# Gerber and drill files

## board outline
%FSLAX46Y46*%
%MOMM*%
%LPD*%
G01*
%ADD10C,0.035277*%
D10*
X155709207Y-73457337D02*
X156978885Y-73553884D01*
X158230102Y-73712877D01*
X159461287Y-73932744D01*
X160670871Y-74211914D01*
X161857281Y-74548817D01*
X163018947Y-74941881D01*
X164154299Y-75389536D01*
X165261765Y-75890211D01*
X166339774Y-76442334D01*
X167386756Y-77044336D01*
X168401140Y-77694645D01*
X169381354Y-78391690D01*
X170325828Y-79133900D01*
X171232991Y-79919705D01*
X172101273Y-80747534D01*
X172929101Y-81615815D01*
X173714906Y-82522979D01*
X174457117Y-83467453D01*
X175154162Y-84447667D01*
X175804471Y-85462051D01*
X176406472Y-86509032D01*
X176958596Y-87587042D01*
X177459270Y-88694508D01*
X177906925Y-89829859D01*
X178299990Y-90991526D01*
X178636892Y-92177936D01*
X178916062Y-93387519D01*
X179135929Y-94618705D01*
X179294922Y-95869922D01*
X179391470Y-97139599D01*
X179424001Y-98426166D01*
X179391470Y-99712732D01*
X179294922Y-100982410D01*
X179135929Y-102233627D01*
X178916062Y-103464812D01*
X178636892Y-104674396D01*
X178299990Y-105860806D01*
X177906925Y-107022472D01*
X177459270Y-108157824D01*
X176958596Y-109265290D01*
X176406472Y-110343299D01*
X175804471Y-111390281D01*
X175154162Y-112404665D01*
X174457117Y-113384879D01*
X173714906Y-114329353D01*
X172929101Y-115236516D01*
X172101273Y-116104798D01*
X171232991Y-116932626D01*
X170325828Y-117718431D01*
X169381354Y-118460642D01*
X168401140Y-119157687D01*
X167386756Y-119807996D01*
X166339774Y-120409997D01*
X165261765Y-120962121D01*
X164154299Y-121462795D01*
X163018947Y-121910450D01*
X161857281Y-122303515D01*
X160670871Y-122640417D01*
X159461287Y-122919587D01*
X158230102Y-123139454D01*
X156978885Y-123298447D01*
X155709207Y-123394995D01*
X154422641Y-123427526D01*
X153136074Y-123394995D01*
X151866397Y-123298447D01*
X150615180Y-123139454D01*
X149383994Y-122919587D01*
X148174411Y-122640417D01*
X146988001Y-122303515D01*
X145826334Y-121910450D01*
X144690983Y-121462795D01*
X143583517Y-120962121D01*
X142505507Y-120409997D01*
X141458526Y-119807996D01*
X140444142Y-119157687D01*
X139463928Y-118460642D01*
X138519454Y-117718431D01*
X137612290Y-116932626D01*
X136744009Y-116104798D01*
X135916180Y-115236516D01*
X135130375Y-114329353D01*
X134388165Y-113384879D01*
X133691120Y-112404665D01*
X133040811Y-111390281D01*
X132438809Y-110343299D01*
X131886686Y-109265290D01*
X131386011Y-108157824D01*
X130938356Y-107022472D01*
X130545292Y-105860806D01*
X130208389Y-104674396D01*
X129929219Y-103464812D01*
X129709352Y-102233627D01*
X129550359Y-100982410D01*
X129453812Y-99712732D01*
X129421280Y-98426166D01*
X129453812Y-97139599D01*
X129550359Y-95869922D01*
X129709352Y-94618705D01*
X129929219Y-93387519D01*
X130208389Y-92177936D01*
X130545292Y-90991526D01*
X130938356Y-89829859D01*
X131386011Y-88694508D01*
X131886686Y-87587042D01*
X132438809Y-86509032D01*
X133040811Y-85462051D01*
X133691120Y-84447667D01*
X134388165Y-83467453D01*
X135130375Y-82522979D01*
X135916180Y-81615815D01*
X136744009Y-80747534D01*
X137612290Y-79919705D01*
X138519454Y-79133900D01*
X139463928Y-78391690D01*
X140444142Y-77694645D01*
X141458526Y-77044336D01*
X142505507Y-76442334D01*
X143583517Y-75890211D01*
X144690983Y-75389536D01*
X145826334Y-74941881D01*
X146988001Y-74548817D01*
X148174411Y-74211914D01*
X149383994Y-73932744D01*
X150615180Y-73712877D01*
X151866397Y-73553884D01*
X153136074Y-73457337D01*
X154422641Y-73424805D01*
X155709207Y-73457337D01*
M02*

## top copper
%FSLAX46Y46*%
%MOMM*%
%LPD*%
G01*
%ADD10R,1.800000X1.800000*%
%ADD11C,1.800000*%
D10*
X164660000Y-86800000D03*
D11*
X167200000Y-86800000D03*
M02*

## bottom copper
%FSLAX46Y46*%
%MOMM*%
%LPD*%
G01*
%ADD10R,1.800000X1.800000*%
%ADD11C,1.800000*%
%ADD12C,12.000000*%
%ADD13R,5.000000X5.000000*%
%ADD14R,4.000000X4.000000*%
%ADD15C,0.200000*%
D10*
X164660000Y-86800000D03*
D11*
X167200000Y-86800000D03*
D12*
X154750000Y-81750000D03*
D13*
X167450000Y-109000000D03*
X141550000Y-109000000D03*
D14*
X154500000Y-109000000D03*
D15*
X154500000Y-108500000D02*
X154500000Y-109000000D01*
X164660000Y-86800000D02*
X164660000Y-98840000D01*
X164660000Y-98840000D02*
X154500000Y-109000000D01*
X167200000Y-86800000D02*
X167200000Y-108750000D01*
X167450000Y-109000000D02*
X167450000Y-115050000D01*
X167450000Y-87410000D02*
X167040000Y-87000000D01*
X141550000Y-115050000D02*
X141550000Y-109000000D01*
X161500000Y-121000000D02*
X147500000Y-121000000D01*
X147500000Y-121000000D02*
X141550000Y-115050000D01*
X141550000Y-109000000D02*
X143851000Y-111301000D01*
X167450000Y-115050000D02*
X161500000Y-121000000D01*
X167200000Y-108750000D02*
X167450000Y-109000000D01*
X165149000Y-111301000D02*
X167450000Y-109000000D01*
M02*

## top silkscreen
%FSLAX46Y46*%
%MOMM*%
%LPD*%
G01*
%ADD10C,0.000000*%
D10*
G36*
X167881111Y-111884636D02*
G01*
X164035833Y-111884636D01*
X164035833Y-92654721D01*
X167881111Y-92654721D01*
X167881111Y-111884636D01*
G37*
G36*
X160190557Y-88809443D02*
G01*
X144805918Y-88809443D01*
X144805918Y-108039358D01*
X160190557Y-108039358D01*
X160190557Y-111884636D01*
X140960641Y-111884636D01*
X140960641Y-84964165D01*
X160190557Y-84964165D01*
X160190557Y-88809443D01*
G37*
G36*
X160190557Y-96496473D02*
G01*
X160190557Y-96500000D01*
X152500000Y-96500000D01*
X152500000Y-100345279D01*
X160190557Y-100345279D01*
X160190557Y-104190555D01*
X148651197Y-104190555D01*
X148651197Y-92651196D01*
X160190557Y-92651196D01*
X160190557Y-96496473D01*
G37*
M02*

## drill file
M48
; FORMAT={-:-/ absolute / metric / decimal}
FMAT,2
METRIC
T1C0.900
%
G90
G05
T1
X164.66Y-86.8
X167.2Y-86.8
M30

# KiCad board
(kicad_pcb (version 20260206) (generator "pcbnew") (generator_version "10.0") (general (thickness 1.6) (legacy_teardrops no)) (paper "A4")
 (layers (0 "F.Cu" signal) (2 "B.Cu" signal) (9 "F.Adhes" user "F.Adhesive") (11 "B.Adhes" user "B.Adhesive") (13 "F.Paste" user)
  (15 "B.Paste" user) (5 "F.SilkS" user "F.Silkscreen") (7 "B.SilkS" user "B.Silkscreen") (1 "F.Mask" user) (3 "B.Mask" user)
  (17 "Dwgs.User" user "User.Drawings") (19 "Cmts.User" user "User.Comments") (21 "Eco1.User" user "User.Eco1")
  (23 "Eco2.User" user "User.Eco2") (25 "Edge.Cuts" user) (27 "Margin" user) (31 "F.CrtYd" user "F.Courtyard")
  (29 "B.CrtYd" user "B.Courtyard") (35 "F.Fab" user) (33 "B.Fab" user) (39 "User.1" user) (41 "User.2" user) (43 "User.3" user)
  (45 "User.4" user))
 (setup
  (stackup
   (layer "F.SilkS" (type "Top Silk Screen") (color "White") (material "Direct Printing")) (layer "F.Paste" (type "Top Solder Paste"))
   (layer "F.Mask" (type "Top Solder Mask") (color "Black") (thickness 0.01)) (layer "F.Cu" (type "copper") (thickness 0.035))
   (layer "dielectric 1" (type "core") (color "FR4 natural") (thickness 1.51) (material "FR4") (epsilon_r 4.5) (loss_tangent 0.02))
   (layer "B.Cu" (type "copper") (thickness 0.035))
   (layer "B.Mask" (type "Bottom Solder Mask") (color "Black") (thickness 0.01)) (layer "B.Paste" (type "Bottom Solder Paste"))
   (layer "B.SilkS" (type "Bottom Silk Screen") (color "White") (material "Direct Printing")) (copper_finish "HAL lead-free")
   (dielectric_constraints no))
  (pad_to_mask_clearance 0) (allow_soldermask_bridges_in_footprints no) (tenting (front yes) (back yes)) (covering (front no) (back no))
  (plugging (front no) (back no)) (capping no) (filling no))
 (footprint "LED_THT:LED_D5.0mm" (layer "F.Cu") (at 164.66 86.8)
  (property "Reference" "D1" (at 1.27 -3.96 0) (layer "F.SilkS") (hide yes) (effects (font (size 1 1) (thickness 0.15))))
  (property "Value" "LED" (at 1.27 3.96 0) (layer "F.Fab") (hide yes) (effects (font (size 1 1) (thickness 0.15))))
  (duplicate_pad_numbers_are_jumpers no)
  (pad "1" thru_hole rect (at 0 0) (size 1.8 1.8) (drill 0.9) (layers "*.Cu" "*.Mask") (remove_unused_layers no) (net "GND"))
  (pad "2" thru_hole circle (at 2.54 0) (size 1.8 1.8) (drill 0.9) (layers "*.Cu" "*.Mask") (remove_unused_layers no) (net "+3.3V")))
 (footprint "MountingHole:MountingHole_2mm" (layer "B.Cu") (at 154.75 81.75 180)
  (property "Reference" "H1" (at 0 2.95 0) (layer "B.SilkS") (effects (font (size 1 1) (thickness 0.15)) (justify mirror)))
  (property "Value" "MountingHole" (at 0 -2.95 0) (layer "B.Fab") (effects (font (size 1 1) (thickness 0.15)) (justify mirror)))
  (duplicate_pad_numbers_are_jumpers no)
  (pad "" smd circle (at 0 0 180) (size 12 12) (layers "B.Cu" "B.Mask" "B.Paste") (thermal_bridge_angle 90)))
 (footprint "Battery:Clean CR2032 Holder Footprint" (layer "B.Cu") (at 154.5 109 180)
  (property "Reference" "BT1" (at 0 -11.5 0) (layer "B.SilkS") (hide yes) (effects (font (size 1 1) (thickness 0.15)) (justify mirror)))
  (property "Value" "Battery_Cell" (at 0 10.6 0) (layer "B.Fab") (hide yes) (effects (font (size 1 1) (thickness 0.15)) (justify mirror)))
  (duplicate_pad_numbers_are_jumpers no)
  (pad "1" smd rect (at -12.95 0 180) (size 5 5) (layers "B.Cu" "B.Mask" "B.Paste") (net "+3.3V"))
  (pad "1" smd rect (at 12.95 0 180) (size 5 5) (layers "B.Cu" "B.Mask" "B.Paste") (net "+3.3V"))
  (pad "2" smd rect (at 0 0 180) (size 4 4) (layers "B.Cu" "B.Mask" "B.Paste") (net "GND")))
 (gr_poly
  (pts (xy 167.881111 111.884636) (xy 164.035833 111.884636) (xy 164.035833 92.654721) (xy 167.881111 92.654721))
  (stroke (width 0) (type solid)) (fill yes) (layer "F.SilkS"))
 (gr_poly
  (pts (xy 160.190557 88.809443) (xy 144.805918 88.809443) (xy 144.805918 108.039358) (xy 160.190557 108.039358) (xy 160.190557 111.884636)
   (xy 140.960641 111.884636) (xy 140.960641 84.964165) (xy 160.190557 84.964165))
  (stroke (width 0) (type solid)) (fill yes) (layer "F.SilkS"))
 (gr_poly
  (pts (xy 160.190557 96.496473) (xy 160.190557 96.5) (xy 152.5 96.5) (xy 152.5 100.345279) (xy 160.190557 100.345279)
   (xy 160.190557 104.190555) (xy 148.651197 104.190555) (xy 148.651197 92.651196) (xy 160.190557 92.651196))
  (stroke (width 0) (type solid)) (fill yes) (layer "F.SilkS"))
 (gr_poly
  (pts (xy 155.709207 73.457337) (xy 156.978885 73.553884) (xy 158.230102 73.712877) (xy 159.461287 73.932744) (xy 160.670871 74.211914)
   (xy 161.857281 74.548817) (xy 163.018947 74.941881) (xy 164.154299 75.389536) (xy 165.261765 75.890211) (xy 166.339774 76.442334)
   (xy 167.386756 77.044336) (xy 168.40114 77.694645) (xy 169.381354 78.39169) (xy 170.325828 79.1339) (xy 171.232991 79.919705)
   (xy 172.101273 80.747534) (xy 172.929101 81.615815) (xy 173.714906 82.522979) (xy 174.457117 83.467453) (xy 175.154162 84.447667)
   (xy 175.804471 85.462051) (xy 176.406472 86.509032) (xy 176.958596 87.587042) (xy 177.45927 88.694508) (xy 177.906925 89.829859)
   (xy 178.29999 90.991526) (xy 178.636892 92.177936) (xy 178.916062 93.387519) (xy 179.135929 94.618705) (xy 179.294922 95.869922)
   (xy 179.39147 97.139599) (xy 179.424001 98.426166) (xy 179.39147 99.712732) (xy 179.294922 100.98241) (xy 179.135929 102.233627)
   (xy 178.916062 103.464812) (xy 178.636892 104.674396) (xy 178.29999 105.860806) (xy 177.906925 107.022472) (xy 177.45927 108.157824)
   (xy 176.958596 109.26529) (xy 176.406472 110.343299) (xy 175.804471 111.390281) (xy 175.154162 112.404665) (xy 174.457117 113.384879)
   (xy 173.714906 114.329353) (xy 172.929101 115.236516) (xy 172.101273 116.104798) (xy 171.232991 116.932626) (xy 170.325828 117.718431)
   (xy 169.381354 118.460642) (xy 168.40114 119.157687) (xy 167.386756 119.807996) (xy 166.339774 120.409997) (xy 165.261765 120.962121)
   (xy 164.154299 121.462795) (xy 163.018947 121.91045) (xy 161.857281 122.303515) (xy 160.670871 122.640417) (xy 159.461287 122.919587)
   (xy 158.230102 123.139454) (xy 156.978885 123.298447) (xy 155.709207 123.394995) (xy 154.422641 123.427526) (xy 153.136074 123.394995)
   (xy 151.866397 123.298447) (xy 150.61518 123.139454) (xy 149.383994 122.919587) (xy 148.174411 122.640417) (xy 146.988001 122.303515)
   (xy 145.826334 121.91045) (xy 144.690983 121.462795) (xy 143.583517 120.962121) (xy 142.505507 120.409997) (xy 141.458526 119.807996)
   (xy 140.444142 119.157687) (xy 139.463928 118.460642) (xy 138.519454 117.718431) (xy 137.61229 116.932626) (xy 136.744009 116.104798)
   (xy 135.91618 115.236516) (xy 135.130375 114.329353) (xy 134.388165 113.384879) (xy 133.69112 112.404665) (xy 133.040811 111.390281)
   (xy 132.438809 110.343299) (xy 131.886686 109.26529) (xy 131.386011 108.157824) (xy 130.938356 107.022472) (xy 130.545292 105.860806)
   (xy 130.208389 104.674396) (xy 129.929219 103.464812) (xy 129.709352 102.233627) (xy 129.550359 100.98241) (xy 129.453812 99.712732)
   (xy 129.42128 98.426166) (xy 129.453812 97.139599) (xy 129.550359 95.869922) (xy 129.709352 94.618705) (xy 129.929219 93.387519)
   (xy 130.208389 92.177936) (xy 130.545292 90.991526) (xy 130.938356 89.829859) (xy 131.386011 88.694508) (xy 131.886686 87.587042)
   (xy 132.438809 86.509032) (xy 133.040811 85.462051) (xy 133.69112 84.447667) (xy 134.388165 83.467453) (xy 135.130375 82.522979)
   (xy 135.91618 81.615815) (xy 136.744009 80.747534) (xy 137.61229 79.919705) (xy 138.519454 79.1339) (xy 139.463928 78.39169)
   (xy 140.444142 77.694645) (xy 141.458526 77.044336) (xy 142.505507 76.442334) (xy 143.583517 75.890211) (xy 144.690983 75.389536)
   (xy 145.826334 74.941881) (xy 146.988001 74.548817) (xy 148.174411 74.211914) (xy 149.383994 73.932744) (xy 150.61518 73.712877)
   (xy 151.866397 73.553884) (xy 153.136074 73.457337) (xy 154.422641 73.424805))
  (stroke (width 0.035277) (type solid) (color 229 36 33 1)) (fill no) (layer "Edge.Cuts"))
 (segment (start 154.5 108.5) (end 154.5 109) (width 0.2) (layer "B.Cu") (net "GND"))
 (segment (start 164.66 86.8) (end 164.66 98.84) (width 0.2) (layer "B.Cu") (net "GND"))
 (segment (start 164.66 98.84) (end 154.5 109) (width 0.2) (layer "B.Cu") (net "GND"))
 (segment (start 167.2 86.8) (end 167.2 108.75) (width 0.2) (layer "B.Cu") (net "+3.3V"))
 (segment (start 167.45 109) (end 167.45 115.05) (width 0.2) (layer "B.Cu") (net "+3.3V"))
 (segment (start 167.45 87.41) (end 167.04 87) (width 0.2) (layer "B.Cu") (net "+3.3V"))
 (segment (start 141.55 115.05) (end 141.55 109) (width 0.2) (layer "B.Cu") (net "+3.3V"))
 (segment (start 161.5 121) (end 147.5 121) (width 0.2) (layer "B.Cu") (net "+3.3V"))
 (segment (start 147.5 121) (end 141.55 115.05) (width 0.2) (layer "B.Cu") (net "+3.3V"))
 (segment (start 141.55 109) (end 143.851 111.301) (width 0.2) (layer "B.Cu") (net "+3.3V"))
 (segment (start 167.45 115.05) (end 161.5 121) (width 0.2) (layer "B.Cu") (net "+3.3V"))
 (segment (start 167.2 108.75) (end 167.45 109) (width 0.2) (layer "B.Cu") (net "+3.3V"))
 (segment (start 165.149 111.301) (end 167.45 109) (width 0.2) (layer "B.Cu") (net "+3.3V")))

